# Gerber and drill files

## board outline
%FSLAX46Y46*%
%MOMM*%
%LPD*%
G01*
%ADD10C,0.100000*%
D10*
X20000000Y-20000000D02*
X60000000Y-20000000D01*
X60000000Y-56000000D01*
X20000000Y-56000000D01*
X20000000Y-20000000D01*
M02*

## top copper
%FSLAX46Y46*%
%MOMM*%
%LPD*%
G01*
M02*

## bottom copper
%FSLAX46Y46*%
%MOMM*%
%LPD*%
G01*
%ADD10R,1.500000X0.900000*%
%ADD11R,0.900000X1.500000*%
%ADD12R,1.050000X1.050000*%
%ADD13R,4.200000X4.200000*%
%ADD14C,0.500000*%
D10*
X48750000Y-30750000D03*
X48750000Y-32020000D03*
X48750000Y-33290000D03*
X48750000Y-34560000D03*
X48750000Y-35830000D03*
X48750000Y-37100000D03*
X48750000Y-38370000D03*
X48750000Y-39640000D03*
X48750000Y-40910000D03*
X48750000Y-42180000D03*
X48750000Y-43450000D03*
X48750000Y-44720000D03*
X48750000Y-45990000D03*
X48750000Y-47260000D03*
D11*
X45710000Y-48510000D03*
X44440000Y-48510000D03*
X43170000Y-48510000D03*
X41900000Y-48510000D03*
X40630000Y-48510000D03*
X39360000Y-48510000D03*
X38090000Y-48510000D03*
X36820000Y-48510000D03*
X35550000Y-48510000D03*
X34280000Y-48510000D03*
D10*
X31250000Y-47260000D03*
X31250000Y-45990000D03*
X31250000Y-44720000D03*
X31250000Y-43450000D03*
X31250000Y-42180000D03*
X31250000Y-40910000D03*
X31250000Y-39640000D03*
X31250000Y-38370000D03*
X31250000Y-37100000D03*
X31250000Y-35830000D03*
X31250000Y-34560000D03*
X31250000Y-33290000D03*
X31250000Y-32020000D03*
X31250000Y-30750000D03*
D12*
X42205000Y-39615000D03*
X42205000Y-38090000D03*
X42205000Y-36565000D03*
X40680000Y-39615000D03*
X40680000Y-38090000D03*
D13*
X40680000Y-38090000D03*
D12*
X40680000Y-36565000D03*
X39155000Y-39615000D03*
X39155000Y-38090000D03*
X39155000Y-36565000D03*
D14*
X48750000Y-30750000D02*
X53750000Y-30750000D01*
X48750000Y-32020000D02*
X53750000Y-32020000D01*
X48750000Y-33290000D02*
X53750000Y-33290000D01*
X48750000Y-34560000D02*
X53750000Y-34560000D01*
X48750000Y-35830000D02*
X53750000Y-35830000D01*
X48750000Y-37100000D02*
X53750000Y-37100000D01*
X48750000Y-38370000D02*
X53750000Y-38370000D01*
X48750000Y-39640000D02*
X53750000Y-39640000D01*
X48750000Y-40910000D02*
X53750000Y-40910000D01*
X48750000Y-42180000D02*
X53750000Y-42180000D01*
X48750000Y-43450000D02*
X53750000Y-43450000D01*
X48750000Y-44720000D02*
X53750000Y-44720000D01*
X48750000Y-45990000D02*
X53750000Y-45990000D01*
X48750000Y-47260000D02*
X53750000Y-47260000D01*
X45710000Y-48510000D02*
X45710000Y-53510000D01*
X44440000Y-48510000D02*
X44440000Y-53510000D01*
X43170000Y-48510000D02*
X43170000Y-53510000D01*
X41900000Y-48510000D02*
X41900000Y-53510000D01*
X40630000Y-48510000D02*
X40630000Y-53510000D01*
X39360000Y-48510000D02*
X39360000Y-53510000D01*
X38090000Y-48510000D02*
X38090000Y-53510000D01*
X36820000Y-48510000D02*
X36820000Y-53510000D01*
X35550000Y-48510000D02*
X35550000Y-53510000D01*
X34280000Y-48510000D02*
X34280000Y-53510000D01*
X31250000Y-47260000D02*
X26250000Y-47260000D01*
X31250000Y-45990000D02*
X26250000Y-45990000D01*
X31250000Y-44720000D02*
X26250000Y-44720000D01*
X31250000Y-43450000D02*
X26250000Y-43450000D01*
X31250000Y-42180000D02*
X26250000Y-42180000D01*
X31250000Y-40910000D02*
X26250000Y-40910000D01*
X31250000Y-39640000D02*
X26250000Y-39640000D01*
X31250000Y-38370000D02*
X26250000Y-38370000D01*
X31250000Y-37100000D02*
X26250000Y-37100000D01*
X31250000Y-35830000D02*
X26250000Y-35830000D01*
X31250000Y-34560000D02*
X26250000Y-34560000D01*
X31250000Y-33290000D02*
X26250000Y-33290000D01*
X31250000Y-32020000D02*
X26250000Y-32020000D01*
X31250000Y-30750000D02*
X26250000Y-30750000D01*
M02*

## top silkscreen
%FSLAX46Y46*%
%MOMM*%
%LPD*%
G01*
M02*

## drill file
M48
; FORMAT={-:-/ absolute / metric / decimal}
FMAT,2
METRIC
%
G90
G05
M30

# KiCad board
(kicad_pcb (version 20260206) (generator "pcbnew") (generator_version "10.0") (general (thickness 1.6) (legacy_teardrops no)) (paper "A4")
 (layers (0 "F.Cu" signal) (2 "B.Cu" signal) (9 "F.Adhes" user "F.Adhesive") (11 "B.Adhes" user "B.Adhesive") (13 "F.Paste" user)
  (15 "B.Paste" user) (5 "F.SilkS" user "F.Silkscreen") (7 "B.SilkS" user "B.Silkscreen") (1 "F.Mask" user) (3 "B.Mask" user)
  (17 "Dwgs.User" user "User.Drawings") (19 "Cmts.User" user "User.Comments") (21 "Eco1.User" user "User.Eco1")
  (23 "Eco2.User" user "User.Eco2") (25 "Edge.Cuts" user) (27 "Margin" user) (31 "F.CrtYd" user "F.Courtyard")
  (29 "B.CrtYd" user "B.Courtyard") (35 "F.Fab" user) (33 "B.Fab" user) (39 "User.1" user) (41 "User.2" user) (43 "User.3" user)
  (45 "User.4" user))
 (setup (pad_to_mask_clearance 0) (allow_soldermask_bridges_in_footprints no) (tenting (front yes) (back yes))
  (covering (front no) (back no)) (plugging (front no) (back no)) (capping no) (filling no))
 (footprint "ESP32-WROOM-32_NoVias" (layer "B.Cu") (at 40 39 180)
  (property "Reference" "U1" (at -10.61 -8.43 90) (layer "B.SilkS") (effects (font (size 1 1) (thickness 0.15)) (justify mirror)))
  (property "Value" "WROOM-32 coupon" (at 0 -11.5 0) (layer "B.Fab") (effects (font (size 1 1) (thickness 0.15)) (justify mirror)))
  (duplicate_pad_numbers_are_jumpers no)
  (pad "1" smd rect (at -8.75 8.25 180) (size 1.5 0.9) (layers "B.Cu" "B.Mask" "B.Paste") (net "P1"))
  (pad "2" smd rect (at -8.75 6.98 180) (size 1.5 0.9) (layers "B.Cu" "B.Mask" "B.Paste") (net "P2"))
  (pad "3" smd rect (at -8.75 5.71 180) (size 1.5 0.9) (layers "B.Cu" "B.Mask" "B.Paste") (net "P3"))
  (pad "4" smd rect (at -8.75 4.44 180) (size 1.5 0.9) (layers "B.Cu" "B.Mask" "B.Paste") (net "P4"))
  (pad "5" smd rect (at -8.75 3.17 180) (size 1.5 0.9) (layers "B.Cu" "B.Mask" "B.Paste") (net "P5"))
  (pad "6" smd rect (at -8.75 1.9 180) (size 1.5 0.9) (layers "B.Cu" "B.Mask" "B.Paste") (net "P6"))
  (pad "7" smd rect (at -8.75 0.63 180) (size 1.5 0.9) (layers "B.Cu" "B.Mask" "B.Paste") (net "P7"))
  (pad "8" smd rect (at -8.75 -0.64 180) (size 1.5 0.9) (layers "B.Cu" "B.Mask" "B.Paste") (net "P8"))
  (pad "9" smd rect (at -8.75 -1.91 180) (size 1.5 0.9) (layers "B.Cu" "B.Mask" "B.Paste") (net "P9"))
  (pad "10" smd rect (at -8.75 -3.18 180) (size 1.5 0.9) (layers "B.Cu" "B.Mask" "B.Paste") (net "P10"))
  (pad "11" smd rect (at -8.75 -4.45 180) (size 1.5 0.9) (layers "B.Cu" "B.Mask" "B.Paste") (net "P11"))
  (pad "12" smd rect (at -8.75 -5.72 180) (size 1.5 0.9) (layers "B.Cu" "B.Mask" "B.Paste") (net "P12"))
  (pad "13" smd rect (at -8.75 -6.99 180) (size 1.5 0.9) (layers "B.Cu" "B.Mask" "B.Paste") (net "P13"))
  (pad "14" smd rect (at -8.75 -8.26 180) (size 1.5 0.9) (layers "B.Cu" "B.Mask" "B.Paste") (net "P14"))
  (pad "15" smd rect (at -5.71 -9.51 90) (size 1.5 0.9) (layers "B.Cu" "B.Mask" "B.Paste") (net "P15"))
  (pad "16" smd rect (at -4.44 -9.51 90) (size 1.5 0.9) (layers "B.Cu" "B.Mask" "B.Paste") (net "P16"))
  (pad "17" smd rect (at -3.17 -9.51 90) (size 1.5 0.9) (layers "B.Cu" "B.Mask" "B.Paste") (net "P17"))
  (pad "18" smd rect (at -1.9 -9.51 90) (size 1.5 0.9) (layers "B.Cu" "B.Mask" "B.Paste") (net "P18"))
  (pad "19" smd rect (at -0.63 -9.51 90) (size 1.5 0.9) (layers "B.Cu" "B.Mask" "B.Paste") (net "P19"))
  (pad "20" smd rect (at 0.64 -9.51 90) (size 1.5 0.9) (layers "B.Cu" "B.Mask" "B.Paste") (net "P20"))
  (pad "21" smd rect (at 1.91 -9.51 90) (size 1.5 0.9) (layers "B.Cu" "B.Mask" "B.Paste") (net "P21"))
  (pad "22" smd rect (at 3.18 -9.51 90) (size 1.5 0.9) (layers "B.Cu" "B.Mask" "B.Paste") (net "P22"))
  (pad "23" smd rect (at 4.45 -9.51 90) (size 1.5 0.9) (layers "B.Cu" "B.Mask" "B.Paste") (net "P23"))
  (pad "24" smd rect (at 5.72 -9.51 90) (size 1.5 0.9) (layers "B.Cu" "B.Mask" "B.Paste") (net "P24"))
  (pad "25" smd rect (at 8.75 -8.26 180) (size 1.5 0.9) (layers "B.Cu" "B.Mask" "B.Paste") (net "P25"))
  (pad "26" smd rect (at 8.75 -6.99 180) (size 1.5 0.9) (layers "B.Cu" "B.Mask" "B.Paste") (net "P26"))
  (pad "27" smd rect (at 8.75 -5.72 180) (size 1.5 0.9) (layers "B.Cu" "B.Mask" "B.Paste") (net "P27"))
  (pad "28" smd rect (at 8.75 -4.45 180) (size 1.5 0.9) (layers "B.Cu" "B.Mask" "B.Paste") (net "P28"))
  (pad "29" smd rect (at 8.75 -3.18 180) (size 1.5 0.9) (layers "B.Cu" "B.Mask" "B.Paste") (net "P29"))
  (pad "30" smd rect (at 8.75 -1.91 180) (size 1.5 0.9) (layers "B.Cu" "B.Mask" "B.Paste") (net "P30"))
  (pad "31" smd rect (at 8.75 -0.64 180) (size 1.5 0.9) (layers "B.Cu" "B.Mask" "B.Paste") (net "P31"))
  (pad "32" smd rect (at 8.75 0.63 180) (size 1.5 0.9) (layers "B.Cu" "B.Mask" "B.Paste") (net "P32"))
  (pad "33" smd rect (at 8.75 1.9 180) (size 1.5 0.9) (layers "B.Cu" "B.Mask" "B.Paste") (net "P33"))
  (pad "34" smd rect (at 8.75 3.17 180) (size 1.5 0.9) (layers "B.Cu" "B.Mask" "B.Paste") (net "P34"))
  (pad "35" smd rect (at 8.75 4.44 180) (size 1.5 0.9) (layers "B.Cu" "B.Mask" "B.Paste") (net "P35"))
  (pad "36" smd rect (at 8.75 5.71 180) (size 1.5 0.9) (layers "B.Cu" "B.Mask" "B.Paste") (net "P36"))
  (pad "37" smd rect (at 8.75 6.98 180) (size 1.5 0.9) (layers "B.Cu" "B.Mask" "B.Paste") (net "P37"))
  (pad "38" smd rect (at 8.75 8.25 180) (size 1.5 0.9) (layers "B.Cu" "B.Mask" "B.Paste") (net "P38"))
  (pad "39" smd rect (at -2.205 -0.615 180) (size 1.05 1.05) (layers "B.Cu" "B.Paste"))
  (pad "39" smd rect (at -2.205 0.91 180) (size 1.05 1.05) (layers "B.Cu" "B.Paste"))
  (pad "39" smd rect (at -2.205 2.435 180) (size 1.05 1.05) (layers "B.Cu" "B.Paste"))
  (pad "39" smd rect (at -0.68 -0.615 180) (size 1.05 1.05) (layers "B.Cu" "B.Paste"))
  (pad "39" smd rect (at -0.68 0.91 180) (size 1.05 1.05) (layers "B.Cu" "B.Paste"))
  (pad "39" smd rect (at -0.68 0.91 180) (size 4.2 4.2) (layers "B.Cu" "B.Mask") (zone_connect 2))
  (pad "39" smd rect (at -0.68 2.435 180) (size 1.05 1.05) (layers "B.Cu" "B.Paste"))
  (pad "39" smd rect (at 0.845 -0.615 180) (size 1.05 1.05) (layers "B.Cu" "B.Paste"))
  (pad "39" smd rect (at 0.845 0.91 180) (size 1.05 1.05) (layers "B.Cu" "B.Paste"))
  (pad "39" smd rect (at 0.845 2.435 180) (size 1.05 1.05) (layers "B.Cu" "B.Paste"))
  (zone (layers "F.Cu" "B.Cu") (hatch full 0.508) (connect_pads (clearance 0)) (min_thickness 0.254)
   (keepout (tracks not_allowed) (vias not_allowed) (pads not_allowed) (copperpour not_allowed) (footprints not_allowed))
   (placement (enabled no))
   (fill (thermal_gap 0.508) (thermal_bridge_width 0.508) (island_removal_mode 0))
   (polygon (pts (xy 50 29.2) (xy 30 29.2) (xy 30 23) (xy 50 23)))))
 (gr_rect (start 20 20) (end 60 56) (stroke (width 0.1) (type default)) (fill no) (layer "Edge.Cuts"))
 (segment (start 48.75 30.75) (end 53.75 30.75) (width 0.5) (layer "B.Cu") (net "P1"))
 (segment (start 48.75 32.02) (end 53.75 32.02) (width 0.5) (layer "B.Cu") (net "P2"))
 (segment (start 48.75 33.29) (end 53.75 33.29) (width 0.5) (layer "B.Cu") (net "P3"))
 (segment (start 48.75 34.56) (end 53.75 34.56) (width 0.5) (layer "B.Cu") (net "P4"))
 (segment (start 48.75 35.83) (end 53.75 35.83) (width 0.5) (layer "B.Cu") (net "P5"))
 (segment (start 48.75 37.1) (end 53.75 37.1) (width 0.5) (layer "B.Cu") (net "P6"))
 (segment (start 48.75 38.37) (end 53.75 38.37) (width 0.5) (layer "B.Cu") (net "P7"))
 (segment (start 48.75 39.64) (end 53.75 39.64) (width 0.5) (layer "B.Cu") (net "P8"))
 (segment (start 48.75 40.91) (end 53.75 40.91) (width 0.5) (layer "B.Cu") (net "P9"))
 (segment (start 48.75 42.18) (end 53.75 42.18) (width 0.5) (layer "B.Cu") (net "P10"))
 (segment (start 48.75 43.45) (end 53.75 43.45) (width 0.5) (layer "B.Cu") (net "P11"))
 (segment (start 48.75 44.72) (end 53.75 44.72) (width 0.5) (layer "B.Cu") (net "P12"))
 (segment (start 48.75 45.99) (end 53.75 45.99) (width 0.5) (layer "B.Cu") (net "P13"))
 (segment (start 48.75 47.26) (end 53.75 47.26) (width 0.5) (layer "B.Cu") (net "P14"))
 (segment (start 45.71 48.51) (end 45.71 53.51) (width 0.5) (layer "B.Cu") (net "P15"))
 (segment (start 44.44 48.51) (end 44.44 53.51) (width 0.5) (layer "B.Cu") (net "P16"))
 (segment (start 43.17 48.51) (end 43.17 53.51) (width 0.5) (layer "B.Cu") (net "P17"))
 (segment (start 41.9 48.51) (end 41.9 53.51) (width 0.5) (layer "B.Cu") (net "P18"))
 (segment (start 40.63 48.51) (end 40.63 53.51) (width 0.5) (layer "B.Cu") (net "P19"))
 (segment (start 39.36 48.51) (end 39.36 53.51) (width 0.5) (layer "B.Cu") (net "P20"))
 (segment (start 38.09 48.51) (end 38.09 53.51) (width 0.5) (layer "B.Cu") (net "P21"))
 (segment (start 36.82 48.51) (end 36.82 53.51) (width 0.5) (layer "B.Cu") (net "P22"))
 (segment (start 35.55 48.51) (end 35.55 53.51) (width 0.5) (layer "B.Cu") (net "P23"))
 (segment (start 34.28 48.51) (end 34.28 53.51) (width 0.5) (layer "B.Cu") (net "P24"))
 (segment (start 31.25 47.26) (end 26.25 47.26) (width 0.5) (layer "B.Cu") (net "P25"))
 (segment (start 31.25 45.99) (end 26.25 45.99) (width 0.5) (layer "B.Cu") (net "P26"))
 (segment (start 31.25 44.72) (end 26.25 44.72) (width 0.5) (layer "B.Cu") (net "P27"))
 (segment (start 31.25 43.45) (end 26.25 43.45) (width 0.5) (layer "B.Cu") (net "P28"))
 (segment (start 31.25 42.18) (end 26.25 42.18) (width 0.5) (layer "B.Cu") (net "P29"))
 (segment (start 31.25 40.91) (end 26.25 40.91) (width 0.5) (layer "B.Cu") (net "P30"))
 (segment (start 31.25 39.64) (end 26.25 39.64) (width 0.5) (layer "B.Cu") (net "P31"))
 (segment (start 31.25 38.37) (end 26.25 38.37) (width 0.5) (layer "B.Cu") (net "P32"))
 (segment (start 31.25 37.1) (end 26.25 37.1) (width 0.5) (layer "B.Cu") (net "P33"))
 (segment (start 31.25 35.83) (end 26.25 35.83) (width 0.5) (layer "B.Cu") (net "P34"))
 (segment (start 31.25 34.56) (end 26.25 34.56) (width 0.5) (layer "B.Cu") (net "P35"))
 (segment (start 31.25 33.29) (end 26.25 33.29) (width 0.5) (layer "B.Cu") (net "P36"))
 (segment (start 31.25 32.02) (end 26.25 32.02) (width 0.5) (layer "B.Cu") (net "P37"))
 (segment (start 31.25 30.75) (end 26.25 30.75) (width 0.5) (layer "B.Cu") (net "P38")))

